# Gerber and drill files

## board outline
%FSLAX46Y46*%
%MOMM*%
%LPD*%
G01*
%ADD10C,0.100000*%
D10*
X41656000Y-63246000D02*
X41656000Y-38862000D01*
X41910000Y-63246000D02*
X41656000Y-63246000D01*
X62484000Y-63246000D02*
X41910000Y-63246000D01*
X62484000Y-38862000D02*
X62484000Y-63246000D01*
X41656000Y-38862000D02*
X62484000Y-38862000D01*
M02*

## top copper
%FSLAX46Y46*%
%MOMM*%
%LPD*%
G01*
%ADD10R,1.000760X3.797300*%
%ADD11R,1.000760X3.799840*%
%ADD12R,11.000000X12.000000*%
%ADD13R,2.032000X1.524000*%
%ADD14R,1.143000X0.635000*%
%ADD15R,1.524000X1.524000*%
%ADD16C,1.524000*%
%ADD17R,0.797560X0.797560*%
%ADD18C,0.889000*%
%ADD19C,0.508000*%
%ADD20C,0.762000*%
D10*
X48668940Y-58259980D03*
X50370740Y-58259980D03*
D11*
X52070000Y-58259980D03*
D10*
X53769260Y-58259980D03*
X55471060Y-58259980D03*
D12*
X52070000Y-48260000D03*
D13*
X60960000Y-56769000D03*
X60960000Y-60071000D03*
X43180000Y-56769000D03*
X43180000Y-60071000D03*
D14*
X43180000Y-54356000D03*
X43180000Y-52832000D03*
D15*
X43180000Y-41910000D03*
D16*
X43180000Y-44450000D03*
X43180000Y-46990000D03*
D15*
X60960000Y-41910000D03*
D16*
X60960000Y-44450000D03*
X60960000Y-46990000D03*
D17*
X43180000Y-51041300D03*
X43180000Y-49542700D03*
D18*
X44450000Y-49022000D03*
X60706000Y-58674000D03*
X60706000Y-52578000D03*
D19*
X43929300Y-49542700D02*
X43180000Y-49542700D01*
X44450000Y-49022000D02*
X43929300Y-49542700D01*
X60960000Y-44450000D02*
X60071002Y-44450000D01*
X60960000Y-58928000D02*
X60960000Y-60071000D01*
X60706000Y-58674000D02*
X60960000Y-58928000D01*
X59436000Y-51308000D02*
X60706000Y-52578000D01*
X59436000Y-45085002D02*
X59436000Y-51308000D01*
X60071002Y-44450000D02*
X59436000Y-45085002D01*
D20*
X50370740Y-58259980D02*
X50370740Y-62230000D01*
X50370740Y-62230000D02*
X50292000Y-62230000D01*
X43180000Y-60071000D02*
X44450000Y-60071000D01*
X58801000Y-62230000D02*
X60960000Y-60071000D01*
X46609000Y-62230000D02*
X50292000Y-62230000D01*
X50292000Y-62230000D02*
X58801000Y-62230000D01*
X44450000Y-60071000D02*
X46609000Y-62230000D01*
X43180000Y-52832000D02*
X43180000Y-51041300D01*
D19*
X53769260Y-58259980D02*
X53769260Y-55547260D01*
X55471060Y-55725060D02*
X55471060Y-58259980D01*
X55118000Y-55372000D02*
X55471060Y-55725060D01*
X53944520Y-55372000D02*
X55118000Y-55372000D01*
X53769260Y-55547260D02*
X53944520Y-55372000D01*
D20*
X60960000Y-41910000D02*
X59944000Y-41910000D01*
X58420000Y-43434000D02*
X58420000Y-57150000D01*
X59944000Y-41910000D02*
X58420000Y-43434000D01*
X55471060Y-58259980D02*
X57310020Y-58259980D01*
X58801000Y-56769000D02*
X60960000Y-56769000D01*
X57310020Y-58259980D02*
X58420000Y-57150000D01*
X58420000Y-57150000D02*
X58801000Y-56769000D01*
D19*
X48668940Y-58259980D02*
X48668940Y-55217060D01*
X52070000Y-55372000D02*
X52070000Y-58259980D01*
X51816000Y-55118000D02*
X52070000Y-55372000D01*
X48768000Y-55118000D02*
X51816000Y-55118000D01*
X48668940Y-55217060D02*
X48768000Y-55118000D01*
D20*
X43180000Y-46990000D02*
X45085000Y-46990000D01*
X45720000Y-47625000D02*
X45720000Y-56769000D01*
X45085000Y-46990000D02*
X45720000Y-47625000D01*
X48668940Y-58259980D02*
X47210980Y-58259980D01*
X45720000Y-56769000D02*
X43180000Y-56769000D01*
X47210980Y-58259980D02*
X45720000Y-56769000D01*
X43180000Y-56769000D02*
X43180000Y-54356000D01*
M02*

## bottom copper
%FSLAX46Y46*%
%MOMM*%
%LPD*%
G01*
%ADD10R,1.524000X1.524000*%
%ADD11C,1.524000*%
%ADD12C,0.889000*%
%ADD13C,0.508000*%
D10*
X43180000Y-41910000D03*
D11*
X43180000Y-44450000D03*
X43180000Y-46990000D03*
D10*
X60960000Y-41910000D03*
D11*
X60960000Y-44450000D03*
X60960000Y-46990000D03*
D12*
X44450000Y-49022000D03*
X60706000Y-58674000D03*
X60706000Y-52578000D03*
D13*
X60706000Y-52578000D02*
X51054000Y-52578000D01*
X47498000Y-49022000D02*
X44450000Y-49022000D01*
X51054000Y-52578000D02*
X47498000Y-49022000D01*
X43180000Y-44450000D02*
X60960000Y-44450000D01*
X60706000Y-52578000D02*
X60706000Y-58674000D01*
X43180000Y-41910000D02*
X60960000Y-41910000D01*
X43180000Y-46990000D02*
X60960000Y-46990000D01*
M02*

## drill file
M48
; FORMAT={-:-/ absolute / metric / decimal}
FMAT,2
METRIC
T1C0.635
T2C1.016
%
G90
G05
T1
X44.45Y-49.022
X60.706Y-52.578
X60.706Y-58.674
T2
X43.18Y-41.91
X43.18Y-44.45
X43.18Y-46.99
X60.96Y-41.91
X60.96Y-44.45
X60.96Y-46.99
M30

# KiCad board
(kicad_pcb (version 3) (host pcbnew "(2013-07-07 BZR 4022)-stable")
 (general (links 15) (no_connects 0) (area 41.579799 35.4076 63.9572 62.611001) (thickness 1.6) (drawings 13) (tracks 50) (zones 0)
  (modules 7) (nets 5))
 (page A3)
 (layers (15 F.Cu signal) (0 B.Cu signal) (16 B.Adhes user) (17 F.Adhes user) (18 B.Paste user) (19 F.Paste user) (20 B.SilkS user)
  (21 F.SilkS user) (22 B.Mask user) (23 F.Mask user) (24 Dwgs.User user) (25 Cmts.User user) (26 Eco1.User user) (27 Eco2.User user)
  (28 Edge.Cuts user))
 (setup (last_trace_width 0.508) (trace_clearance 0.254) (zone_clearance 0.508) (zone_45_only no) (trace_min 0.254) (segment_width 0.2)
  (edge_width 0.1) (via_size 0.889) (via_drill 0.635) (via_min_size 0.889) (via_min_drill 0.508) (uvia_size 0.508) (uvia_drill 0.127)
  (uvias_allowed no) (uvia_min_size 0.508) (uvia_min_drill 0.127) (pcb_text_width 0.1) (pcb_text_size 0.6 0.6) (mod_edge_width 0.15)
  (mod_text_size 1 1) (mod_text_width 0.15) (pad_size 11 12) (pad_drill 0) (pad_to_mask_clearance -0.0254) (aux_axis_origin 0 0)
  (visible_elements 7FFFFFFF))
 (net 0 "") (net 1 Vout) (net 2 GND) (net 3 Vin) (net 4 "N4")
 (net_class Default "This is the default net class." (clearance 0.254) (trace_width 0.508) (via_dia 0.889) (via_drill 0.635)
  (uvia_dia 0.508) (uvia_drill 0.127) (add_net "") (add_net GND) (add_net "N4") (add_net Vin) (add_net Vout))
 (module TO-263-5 (layer F.Cu) (at 52.07 45.72)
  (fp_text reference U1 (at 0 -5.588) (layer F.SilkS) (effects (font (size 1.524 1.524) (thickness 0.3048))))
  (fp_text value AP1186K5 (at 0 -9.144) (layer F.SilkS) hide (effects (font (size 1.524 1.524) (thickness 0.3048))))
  (pad 1 smd rect (at -3.40106 12.53998 90) (size 3.7973 1.00076) (layers F.Cu F.Paste F.Mask) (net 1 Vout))
  (pad 2 smd rect (at -1.69926 12.53998 90) (size 3.7973 1.00076) (layers F.Cu F.Paste F.Mask) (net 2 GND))
  (pad 3 smd rect (at 0 12.53998 90) (size 3.79984 1.00076) (layers F.Cu F.Paste F.Mask) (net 1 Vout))
  (pad 4 smd rect (at 1.69926 12.53998 90) (size 3.7973 1.00076) (layers F.Cu F.Paste F.Mask) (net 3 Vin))
  (pad 5 smd rect (at 3.40106 12.53998 90) (size 3.7973 1.00076) (layers F.Cu F.Paste F.Mask) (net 3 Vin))
  (pad 6 smd rect (at 0 2.54 180) (size 11 12) (layers F.Cu F.Paste F.Mask) (clearance 0.254)))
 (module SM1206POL (layer F.Cu) (at 60.96 58.42 270)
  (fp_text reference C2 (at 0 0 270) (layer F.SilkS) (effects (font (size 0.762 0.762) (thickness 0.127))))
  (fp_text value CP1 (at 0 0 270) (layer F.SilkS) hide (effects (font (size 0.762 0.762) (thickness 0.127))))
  (pad 1 smd rect (at -1.651 0 270) (size 1.524 2.032) (layers F.Cu F.Paste F.Mask) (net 3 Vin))
  (pad 2 smd rect (at 1.651 0 270) (size 1.524 2.032) (layers F.Cu F.Paste F.Mask) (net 2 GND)))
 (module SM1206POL (layer F.Cu) (at 43.18 58.42 270)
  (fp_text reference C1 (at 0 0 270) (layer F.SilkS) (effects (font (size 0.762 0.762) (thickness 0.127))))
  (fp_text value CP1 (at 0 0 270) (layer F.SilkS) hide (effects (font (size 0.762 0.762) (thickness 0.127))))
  (pad 1 smd rect (at -1.651 0 270) (size 1.524 2.032) (layers F.Cu F.Paste F.Mask) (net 1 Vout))
  (pad 2 smd rect (at 1.651 0 270) (size 1.524 2.032) (layers F.Cu F.Paste F.Mask) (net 2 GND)))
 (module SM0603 (layer F.Cu) (at 43.18 53.594 90)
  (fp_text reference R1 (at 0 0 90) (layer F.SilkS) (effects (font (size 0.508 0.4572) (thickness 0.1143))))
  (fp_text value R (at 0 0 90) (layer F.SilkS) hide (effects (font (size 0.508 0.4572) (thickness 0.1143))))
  (pad 1 smd rect (at -0.762 0 90) (size 0.635 1.143) (layers F.Cu F.Paste F.Mask) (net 1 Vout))
  (pad 2 smd rect (at 0.762 0 90) (size 0.635 1.143) (layers F.Cu F.Paste F.Mask) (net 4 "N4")))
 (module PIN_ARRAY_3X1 (layer F.Cu) (at 43.18 44.45 270)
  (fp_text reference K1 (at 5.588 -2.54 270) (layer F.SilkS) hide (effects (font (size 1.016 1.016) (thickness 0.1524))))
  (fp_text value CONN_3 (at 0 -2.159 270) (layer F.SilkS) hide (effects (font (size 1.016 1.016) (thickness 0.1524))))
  (pad 1 thru_hole rect (at -2.54 0 270) (size 1.524 1.524) (drill 1.016) (layers *.Cu *.Mask F.SilkS) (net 3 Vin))
  (pad 2 thru_hole circle (at 0 0 270) (size 1.524 1.524) (drill 1.016) (layers *.Cu *.Mask F.SilkS) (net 2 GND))
  (pad 3 thru_hole circle (at 2.54 0 270) (size 1.524 1.524) (drill 1.016) (layers *.Cu *.Mask F.SilkS) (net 1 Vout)))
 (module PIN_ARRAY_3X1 (layer F.Cu) (at 60.96 44.45 270)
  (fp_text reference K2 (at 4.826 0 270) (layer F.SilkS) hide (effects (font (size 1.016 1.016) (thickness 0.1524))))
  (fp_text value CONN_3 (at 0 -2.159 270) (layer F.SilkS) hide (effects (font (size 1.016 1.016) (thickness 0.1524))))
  (pad 1 thru_hole rect (at -2.54 0 270) (size 1.524 1.524) (drill 1.016) (layers *.Cu *.Mask F.SilkS) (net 3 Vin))
  (pad 2 thru_hole circle (at 0 0 270) (size 1.524 1.524) (drill 1.016) (layers *.Cu *.Mask F.SilkS) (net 2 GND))
  (pad 3 thru_hole circle (at 2.54 0 270) (size 1.524 1.524) (drill 1.016) (layers *.Cu *.Mask F.SilkS) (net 1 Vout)))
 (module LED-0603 (layer F.Cu) (at 43.18 50.292 90)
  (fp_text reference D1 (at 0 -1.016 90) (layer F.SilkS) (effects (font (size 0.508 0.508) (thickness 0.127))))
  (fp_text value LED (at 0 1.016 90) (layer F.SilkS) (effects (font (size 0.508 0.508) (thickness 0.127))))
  (pad 1 smd rect (at -0.7493 0 90) (size 0.79756 0.79756) (layers F.Cu F.Paste F.Mask) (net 4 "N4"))
  (pad 2 smd rect (at 0.7493 0 90) (size 0.79756 0.79756) (layers F.Cu F.Paste F.Mask) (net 2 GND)))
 (gr_line (start 41.656 63.246) (end 41.656 38.862) (angle 90) (layer Edge.Cuts) (width 0.1))
 (gr_line (start 41.91 63.246) (end 41.656 63.246) (angle 90) (layer Edge.Cuts) (width 0.1))
 (gr_line (start 62.484 63.246) (end 41.91 63.246) (angle 90) (layer Edge.Cuts) (width 0.1))
 (gr_line (start 62.484 38.862) (end 62.484 63.246) (angle 90) (layer Edge.Cuts) (width 0.1))
 (gr_line (start 41.656 38.862) (end 62.484 38.862) (angle 90) (layer Edge.Cuts) (width 0.1))
 (segment (start 60.706 52.578) (end 51.054 52.578) (width 0.508) (layer B.Cu) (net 2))
 (segment (start 43.9293 49.5427) (end 43.18 49.5427) (width 0.508) (layer F.Cu) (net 2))
 (segment (start 44.45 49.022) (end 43.9293 49.5427) (width 0.508) (layer F.Cu) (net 2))
 (via (at 44.45 49.022) (size 0.889) (layers F.Cu B.Cu) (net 2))
 (segment (start 47.498 49.022) (end 44.45 49.022) (width 0.508) (layer B.Cu) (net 2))
 (segment (start 51.054 52.578) (end 47.498 49.022) (width 0.508) (layer B.Cu) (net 2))
 (segment (start 43.18 44.45) (end 60.96 44.45) (width 0.508) (layer B.Cu) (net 2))
 (segment (start 60.96 44.45) (end 60.071002 44.45) (width 0.508) (layer F.Cu) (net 2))
 (segment (start 60.96 58.928) (end 60.96 60.071) (width 0.508) (layer F.Cu) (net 2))
 (segment (start 60.706 58.674) (end 60.96 58.928) (width 0.508) (layer F.Cu) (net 2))
 (via (at 60.706 58.674) (size 0.889) (layers F.Cu B.Cu) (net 2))
 (segment (start 60.706 52.578) (end 60.706 58.674) (width 0.508) (layer B.Cu) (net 2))
 (via (at 60.706 52.578) (size 0.889) (layers F.Cu B.Cu) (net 2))
 (segment (start 59.436 51.308) (end 60.706 52.578) (width 0.508) (layer F.Cu) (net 2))
 (segment (start 59.436 45.085002) (end 59.436 51.308) (width 0.508) (layer F.Cu) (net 2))
 (segment (start 60.071002 44.45) (end 59.436 45.085002) (width 0.508) (layer F.Cu) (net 2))
 (segment (start 50.37074 58.25998) (end 50.37074 62.23) (width 0.762) (layer F.Cu) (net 2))
 (segment (start 50.37074 62.23) (end 50.292 62.23) (width 0.762) (layer F.Cu) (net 2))
 (segment (start 43.18 60.071) (end 44.45 60.071) (width 0.762) (layer F.Cu) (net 2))
 (segment (start 58.801 62.23) (end 60.96 60.071) (width 0.762) (layer F.Cu) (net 2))
 (segment (start 46.609 62.23) (end 50.292 62.23) (width 0.762) (layer F.Cu) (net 2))
 (segment (start 50.292 62.23) (end 58.801 62.23) (width 0.762) (layer F.Cu) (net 2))
 (segment (start 44.45 60.071) (end 46.609 62.23) (width 0.762) (layer F.Cu) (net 2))
 (segment (start 43.18 52.832) (end 43.18 51.0413) (width 0.762) (layer F.Cu) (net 4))
 (segment (start 53.76926 58.25998) (end 53.76926 55.54726) (width 0.508) (layer F.Cu) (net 3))
 (segment (start 55.47106 55.72506) (end 55.47106 58.25998) (width 0.508) (layer F.Cu) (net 3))
 (segment (start 55.118 55.372) (end 55.47106 55.72506) (width 0.508) (layer F.Cu) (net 3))
 (segment (start 53.94452 55.372) (end 55.118 55.372) (width 0.508) (layer F.Cu) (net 3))
 (segment (start 53.76926 55.54726) (end 53.94452 55.372) (width 0.508) (layer F.Cu) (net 3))
 (segment (start 43.18 41.91) (end 60.96 41.91) (width 0.508) (layer B.Cu) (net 3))
 (segment (start 60.96 41.91) (end 59.944 41.91) (width 0.762) (layer F.Cu) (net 3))
 (segment (start 58.42 43.434) (end 58.42 57.15) (width 0.762) (layer F.Cu) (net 3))
 (segment (start 59.944 41.91) (end 58.42 43.434) (width 0.762) (layer F.Cu) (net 3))
 (segment (start 55.47106 58.25998) (end 57.31002 58.25998) (width 0.762) (layer F.Cu) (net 3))
 (segment (start 58.801 56.769) (end 60.96 56.769) (width 0.762) (layer F.Cu) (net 3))
 (segment (start 57.31002 58.25998) (end 58.42 57.15) (width 0.762) (layer F.Cu) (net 3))
 (segment (start 58.42 57.15) (end 58.801 56.769) (width 0.762) (layer F.Cu) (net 3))
 (segment (start 48.66894 58.25998) (end 48.66894 55.21706) (width 0.508) (layer F.Cu) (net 1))
 (segment (start 52.07 55.372) (end 52.07 58.25998) (width 0.508) (layer F.Cu) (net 1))
 (segment (start 51.816 55.118) (end 52.07 55.372) (width 0.508) (layer F.Cu) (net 1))
 (segment (start 48.768 55.118) (end 51.816 55.118) (width 0.508) (layer F.Cu) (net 1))
 (segment (start 48.66894 55.21706) (end 48.768 55.118) (width 0.508) (layer F.Cu) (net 1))
 (segment (start 43.18 46.99) (end 60.96 46.99) (width 0.508) (layer B.Cu) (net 1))
 (segment (start 43.18 46.99) (end 45.085 46.99) (width 0.762) (layer F.Cu) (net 1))
 (segment (start 45.72 47.625) (end 45.72 56.769) (width 0.762) (layer F.Cu) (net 1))
 (segment (start 45.085 46.99) (end 45.72 47.625) (width 0.762) (layer F.Cu) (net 1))
 (segment (start 48.66894 58.25998) (end 47.21098 58.25998) (width 0.762) (layer F.Cu) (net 1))
 (segment (start 45.72 56.769) (end 43.18 56.769) (width 0.762) (layer F.Cu) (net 1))
 (segment (start 47.21098 58.25998) (end 45.72 56.769) (width 0.762) (layer F.Cu) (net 1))
 (segment (start 43.18 56.769) (end 43.18 54.356) (width 0.762) (layer F.Cu) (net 1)))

